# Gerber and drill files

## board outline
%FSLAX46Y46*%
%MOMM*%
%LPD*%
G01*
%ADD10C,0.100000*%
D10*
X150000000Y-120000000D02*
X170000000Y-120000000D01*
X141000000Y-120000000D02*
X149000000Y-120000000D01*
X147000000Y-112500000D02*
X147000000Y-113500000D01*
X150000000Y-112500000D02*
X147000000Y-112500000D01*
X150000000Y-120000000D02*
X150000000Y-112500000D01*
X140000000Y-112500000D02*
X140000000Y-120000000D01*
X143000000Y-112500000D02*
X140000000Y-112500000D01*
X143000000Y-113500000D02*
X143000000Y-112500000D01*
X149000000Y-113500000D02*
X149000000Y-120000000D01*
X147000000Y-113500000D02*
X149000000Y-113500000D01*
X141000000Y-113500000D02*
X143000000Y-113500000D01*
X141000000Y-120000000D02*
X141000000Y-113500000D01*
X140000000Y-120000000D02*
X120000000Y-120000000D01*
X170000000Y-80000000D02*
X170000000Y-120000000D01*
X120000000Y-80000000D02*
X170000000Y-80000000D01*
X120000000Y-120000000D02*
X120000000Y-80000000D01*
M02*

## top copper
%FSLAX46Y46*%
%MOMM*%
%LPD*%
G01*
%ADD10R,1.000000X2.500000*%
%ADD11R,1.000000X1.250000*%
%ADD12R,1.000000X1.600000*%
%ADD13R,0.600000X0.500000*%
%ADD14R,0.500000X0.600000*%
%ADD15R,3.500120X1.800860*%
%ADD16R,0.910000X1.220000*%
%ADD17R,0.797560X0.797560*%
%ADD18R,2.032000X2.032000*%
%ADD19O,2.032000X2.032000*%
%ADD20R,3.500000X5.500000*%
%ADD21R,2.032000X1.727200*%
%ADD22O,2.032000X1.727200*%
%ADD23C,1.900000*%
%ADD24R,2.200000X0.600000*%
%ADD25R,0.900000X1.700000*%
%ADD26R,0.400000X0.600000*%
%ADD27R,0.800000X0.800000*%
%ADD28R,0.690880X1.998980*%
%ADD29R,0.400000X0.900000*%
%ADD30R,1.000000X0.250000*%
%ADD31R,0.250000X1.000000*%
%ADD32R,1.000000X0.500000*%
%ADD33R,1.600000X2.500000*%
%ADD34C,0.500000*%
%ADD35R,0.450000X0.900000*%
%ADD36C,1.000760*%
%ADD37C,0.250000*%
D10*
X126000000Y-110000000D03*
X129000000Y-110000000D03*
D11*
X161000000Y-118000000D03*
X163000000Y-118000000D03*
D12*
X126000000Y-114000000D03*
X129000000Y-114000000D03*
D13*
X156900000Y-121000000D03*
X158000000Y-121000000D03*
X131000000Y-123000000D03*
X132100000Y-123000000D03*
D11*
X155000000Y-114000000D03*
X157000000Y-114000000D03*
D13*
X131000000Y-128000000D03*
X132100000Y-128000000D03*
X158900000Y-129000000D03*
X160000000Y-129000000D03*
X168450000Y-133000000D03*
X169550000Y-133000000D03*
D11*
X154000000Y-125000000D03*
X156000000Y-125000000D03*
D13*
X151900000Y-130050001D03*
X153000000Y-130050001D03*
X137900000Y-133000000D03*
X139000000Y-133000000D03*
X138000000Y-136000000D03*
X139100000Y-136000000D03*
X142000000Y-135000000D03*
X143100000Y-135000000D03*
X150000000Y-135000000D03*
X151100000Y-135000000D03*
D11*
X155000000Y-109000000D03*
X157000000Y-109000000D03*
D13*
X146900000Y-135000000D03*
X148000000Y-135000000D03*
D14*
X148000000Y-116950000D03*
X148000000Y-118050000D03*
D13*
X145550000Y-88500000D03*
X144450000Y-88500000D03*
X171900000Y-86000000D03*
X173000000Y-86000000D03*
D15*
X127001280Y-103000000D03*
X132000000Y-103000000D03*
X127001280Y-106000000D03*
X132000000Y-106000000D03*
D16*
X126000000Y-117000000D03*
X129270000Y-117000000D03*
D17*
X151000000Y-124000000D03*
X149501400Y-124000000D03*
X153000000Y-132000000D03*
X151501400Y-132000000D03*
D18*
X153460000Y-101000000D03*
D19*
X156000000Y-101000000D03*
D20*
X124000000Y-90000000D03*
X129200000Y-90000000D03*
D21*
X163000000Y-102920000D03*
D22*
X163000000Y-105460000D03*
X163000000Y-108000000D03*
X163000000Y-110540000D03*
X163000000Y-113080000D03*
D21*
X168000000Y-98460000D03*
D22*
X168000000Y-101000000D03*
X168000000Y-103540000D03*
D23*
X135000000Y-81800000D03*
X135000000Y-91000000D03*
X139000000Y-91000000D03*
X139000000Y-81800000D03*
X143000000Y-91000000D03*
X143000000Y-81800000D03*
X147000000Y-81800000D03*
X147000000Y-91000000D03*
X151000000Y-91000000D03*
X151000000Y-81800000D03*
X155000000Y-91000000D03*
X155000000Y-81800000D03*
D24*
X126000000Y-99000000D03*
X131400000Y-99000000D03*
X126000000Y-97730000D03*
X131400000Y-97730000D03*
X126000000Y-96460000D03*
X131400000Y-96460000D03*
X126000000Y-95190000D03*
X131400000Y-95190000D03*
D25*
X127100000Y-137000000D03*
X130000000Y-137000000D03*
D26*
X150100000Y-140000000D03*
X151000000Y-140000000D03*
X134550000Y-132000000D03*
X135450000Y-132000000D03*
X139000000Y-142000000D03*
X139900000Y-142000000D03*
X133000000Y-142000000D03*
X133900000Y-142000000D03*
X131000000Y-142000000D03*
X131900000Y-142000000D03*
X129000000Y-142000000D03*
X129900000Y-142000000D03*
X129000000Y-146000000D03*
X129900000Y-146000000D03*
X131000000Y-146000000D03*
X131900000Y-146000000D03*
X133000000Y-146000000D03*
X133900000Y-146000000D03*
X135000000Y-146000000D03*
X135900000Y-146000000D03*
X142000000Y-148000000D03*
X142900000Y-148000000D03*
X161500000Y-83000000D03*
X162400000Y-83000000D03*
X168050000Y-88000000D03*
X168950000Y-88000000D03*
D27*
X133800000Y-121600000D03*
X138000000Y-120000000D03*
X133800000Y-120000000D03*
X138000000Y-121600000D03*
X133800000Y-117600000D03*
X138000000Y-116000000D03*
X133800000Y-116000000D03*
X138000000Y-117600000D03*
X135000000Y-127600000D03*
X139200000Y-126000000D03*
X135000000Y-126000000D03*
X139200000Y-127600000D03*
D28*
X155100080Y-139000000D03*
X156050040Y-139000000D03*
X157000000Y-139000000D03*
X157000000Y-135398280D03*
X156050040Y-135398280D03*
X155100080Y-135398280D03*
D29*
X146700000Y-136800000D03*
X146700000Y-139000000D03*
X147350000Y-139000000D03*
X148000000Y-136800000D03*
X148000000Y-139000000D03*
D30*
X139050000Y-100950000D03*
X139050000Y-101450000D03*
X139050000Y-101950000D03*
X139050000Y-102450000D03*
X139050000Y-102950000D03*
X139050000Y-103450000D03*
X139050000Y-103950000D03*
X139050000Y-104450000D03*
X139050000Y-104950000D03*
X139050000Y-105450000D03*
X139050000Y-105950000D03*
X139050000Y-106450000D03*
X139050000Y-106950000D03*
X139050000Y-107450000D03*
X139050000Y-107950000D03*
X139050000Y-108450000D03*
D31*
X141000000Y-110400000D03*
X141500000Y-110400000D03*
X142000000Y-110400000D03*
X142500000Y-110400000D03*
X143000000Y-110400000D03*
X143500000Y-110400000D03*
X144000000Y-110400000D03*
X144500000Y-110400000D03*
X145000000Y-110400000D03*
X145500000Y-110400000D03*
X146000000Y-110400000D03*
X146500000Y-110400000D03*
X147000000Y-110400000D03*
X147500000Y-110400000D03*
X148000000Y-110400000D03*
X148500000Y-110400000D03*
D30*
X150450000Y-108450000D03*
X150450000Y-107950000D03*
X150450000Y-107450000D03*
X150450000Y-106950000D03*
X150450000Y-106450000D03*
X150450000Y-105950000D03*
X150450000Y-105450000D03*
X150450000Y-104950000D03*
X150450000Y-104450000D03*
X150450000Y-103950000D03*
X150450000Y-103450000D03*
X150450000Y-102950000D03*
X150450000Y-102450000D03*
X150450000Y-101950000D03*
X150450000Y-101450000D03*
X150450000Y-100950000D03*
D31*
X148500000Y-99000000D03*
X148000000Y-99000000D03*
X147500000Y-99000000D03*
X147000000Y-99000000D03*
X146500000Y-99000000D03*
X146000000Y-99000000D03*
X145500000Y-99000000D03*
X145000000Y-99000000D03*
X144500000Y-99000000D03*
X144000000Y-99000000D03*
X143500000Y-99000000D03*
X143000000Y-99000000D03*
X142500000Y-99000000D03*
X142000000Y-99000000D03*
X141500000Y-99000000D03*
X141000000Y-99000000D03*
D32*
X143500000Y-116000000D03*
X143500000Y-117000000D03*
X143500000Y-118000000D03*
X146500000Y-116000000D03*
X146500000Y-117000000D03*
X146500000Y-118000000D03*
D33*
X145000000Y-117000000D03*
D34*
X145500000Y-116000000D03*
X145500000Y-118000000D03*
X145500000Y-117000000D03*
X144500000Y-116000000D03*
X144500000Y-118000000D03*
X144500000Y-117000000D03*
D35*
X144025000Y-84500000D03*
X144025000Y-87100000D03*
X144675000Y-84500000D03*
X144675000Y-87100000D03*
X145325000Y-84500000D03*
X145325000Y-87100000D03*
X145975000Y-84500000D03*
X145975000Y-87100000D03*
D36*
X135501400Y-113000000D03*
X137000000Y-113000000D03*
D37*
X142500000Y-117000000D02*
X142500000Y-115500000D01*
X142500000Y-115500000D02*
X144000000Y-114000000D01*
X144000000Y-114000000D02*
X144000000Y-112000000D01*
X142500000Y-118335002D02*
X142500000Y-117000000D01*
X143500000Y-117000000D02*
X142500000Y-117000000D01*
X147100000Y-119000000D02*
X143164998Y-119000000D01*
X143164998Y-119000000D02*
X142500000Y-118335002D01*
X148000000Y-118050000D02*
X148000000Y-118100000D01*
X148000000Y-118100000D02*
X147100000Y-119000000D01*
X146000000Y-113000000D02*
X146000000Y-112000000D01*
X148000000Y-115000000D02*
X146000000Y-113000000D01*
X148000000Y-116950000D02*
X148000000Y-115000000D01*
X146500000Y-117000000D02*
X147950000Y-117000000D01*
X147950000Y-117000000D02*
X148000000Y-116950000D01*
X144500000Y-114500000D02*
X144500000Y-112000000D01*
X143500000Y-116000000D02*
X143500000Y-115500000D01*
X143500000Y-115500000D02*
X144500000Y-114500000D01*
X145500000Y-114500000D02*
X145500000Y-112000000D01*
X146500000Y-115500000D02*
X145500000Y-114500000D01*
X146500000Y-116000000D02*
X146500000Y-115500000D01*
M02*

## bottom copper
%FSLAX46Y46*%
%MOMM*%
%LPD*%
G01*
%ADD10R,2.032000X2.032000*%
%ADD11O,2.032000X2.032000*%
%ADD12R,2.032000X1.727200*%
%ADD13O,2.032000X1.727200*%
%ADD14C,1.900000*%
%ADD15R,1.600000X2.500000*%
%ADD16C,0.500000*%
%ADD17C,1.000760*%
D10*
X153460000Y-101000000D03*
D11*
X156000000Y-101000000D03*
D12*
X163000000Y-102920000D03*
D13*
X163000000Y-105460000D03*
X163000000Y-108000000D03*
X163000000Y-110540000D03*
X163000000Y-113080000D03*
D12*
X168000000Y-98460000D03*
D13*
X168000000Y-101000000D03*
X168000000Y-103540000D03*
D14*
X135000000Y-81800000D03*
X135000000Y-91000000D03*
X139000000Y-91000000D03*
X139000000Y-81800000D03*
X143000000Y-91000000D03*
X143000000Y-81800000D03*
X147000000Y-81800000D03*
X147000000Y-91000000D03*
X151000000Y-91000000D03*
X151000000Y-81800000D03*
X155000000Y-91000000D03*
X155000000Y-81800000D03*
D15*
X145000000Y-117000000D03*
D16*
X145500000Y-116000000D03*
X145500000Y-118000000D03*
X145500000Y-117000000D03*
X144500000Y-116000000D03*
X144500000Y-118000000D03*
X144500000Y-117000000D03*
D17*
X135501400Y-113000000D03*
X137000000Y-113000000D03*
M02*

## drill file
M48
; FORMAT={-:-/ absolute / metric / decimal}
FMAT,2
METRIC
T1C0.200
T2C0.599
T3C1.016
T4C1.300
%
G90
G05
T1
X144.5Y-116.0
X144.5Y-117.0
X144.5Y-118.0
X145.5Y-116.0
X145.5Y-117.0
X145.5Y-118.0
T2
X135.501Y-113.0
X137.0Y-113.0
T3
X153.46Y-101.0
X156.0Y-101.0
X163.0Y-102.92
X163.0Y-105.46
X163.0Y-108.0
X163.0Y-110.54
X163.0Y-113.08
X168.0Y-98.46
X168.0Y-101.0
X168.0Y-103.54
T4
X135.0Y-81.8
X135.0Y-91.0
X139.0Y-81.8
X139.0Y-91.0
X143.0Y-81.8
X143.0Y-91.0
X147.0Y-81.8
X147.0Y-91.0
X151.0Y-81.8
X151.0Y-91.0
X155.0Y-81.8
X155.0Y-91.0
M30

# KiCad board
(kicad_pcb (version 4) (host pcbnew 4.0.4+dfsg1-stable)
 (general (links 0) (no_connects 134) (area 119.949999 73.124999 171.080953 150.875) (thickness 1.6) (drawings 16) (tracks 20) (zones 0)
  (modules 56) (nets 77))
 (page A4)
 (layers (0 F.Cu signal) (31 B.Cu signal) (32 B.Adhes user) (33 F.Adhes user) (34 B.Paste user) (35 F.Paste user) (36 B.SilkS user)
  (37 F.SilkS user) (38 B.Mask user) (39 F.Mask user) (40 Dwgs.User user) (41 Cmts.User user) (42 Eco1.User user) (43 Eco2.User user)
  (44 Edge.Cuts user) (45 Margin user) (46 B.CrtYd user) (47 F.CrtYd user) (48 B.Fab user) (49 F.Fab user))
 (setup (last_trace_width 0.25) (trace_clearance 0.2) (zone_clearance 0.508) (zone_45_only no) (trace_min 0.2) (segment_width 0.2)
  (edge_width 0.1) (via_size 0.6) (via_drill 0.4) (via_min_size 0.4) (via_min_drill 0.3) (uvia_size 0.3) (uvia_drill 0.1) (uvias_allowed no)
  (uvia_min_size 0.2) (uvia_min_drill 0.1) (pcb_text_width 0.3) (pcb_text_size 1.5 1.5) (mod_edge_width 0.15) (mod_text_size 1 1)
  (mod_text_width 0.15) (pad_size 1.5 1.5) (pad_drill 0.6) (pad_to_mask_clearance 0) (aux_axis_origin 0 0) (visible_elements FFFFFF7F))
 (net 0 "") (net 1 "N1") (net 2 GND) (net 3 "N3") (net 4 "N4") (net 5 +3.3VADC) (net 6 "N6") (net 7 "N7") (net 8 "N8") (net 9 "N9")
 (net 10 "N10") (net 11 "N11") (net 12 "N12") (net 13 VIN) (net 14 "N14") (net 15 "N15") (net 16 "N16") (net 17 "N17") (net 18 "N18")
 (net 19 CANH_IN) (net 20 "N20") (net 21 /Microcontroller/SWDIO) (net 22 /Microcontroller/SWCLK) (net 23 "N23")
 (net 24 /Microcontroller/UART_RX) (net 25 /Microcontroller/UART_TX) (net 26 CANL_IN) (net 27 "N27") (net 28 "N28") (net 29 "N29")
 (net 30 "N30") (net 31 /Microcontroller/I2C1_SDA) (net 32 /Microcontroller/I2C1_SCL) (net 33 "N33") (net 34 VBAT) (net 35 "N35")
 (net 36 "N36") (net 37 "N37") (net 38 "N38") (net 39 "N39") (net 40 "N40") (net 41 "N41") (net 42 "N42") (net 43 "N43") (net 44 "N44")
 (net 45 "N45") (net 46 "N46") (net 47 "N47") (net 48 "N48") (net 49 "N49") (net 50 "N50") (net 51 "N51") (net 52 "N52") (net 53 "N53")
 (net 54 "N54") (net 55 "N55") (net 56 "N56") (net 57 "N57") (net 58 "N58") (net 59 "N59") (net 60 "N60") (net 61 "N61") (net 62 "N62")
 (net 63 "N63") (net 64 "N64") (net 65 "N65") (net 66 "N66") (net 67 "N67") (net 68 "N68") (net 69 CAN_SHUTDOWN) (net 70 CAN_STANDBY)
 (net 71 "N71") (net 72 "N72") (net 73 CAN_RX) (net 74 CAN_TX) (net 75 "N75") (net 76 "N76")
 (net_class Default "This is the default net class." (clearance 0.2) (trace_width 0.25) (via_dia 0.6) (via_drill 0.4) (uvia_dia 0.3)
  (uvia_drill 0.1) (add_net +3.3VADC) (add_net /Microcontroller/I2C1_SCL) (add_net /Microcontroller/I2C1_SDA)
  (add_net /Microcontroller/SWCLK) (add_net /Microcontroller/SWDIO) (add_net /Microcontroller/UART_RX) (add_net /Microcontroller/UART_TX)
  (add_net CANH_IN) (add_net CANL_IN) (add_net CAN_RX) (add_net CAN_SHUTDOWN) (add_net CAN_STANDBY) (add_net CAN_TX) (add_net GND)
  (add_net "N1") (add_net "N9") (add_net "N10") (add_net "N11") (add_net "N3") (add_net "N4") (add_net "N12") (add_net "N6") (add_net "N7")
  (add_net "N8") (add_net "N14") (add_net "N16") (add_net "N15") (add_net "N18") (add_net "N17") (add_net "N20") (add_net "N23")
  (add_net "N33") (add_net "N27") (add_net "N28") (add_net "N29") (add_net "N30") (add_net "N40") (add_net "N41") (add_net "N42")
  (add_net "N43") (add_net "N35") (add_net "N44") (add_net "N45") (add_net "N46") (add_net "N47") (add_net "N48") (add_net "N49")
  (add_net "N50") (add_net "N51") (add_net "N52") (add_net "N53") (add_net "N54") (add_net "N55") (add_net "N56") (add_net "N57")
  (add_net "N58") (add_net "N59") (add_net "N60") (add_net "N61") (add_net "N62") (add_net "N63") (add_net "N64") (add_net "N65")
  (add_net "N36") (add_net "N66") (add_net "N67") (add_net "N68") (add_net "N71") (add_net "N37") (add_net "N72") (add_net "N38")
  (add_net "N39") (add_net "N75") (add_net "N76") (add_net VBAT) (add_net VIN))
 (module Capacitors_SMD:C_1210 (layer F.Cu) (at 127.5 110)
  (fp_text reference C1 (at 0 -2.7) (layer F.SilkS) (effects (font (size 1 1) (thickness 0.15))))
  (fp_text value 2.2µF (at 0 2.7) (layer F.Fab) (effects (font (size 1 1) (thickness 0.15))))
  (pad 1 smd rect (at -1.5 0) (size 1 2.5) (layers F.Cu F.Paste F.Mask) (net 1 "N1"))
  (pad 2 smd rect (at 1.5 0) (size 1 2.5) (layers F.Cu F.Paste F.Mask) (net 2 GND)))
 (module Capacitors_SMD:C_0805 (layer F.Cu) (at 162 118)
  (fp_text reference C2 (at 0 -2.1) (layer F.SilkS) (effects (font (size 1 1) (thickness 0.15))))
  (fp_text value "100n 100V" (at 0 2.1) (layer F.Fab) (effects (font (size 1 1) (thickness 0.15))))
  (pad 1 smd rect (at -1 0) (size 1 1.25) (layers F.Cu F.Paste F.Mask) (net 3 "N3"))
  (pad 2 smd rect (at 1 0) (size 1 1.25) (layers F.Cu F.Paste F.Mask) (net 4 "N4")))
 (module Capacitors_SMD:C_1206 (layer F.Cu) (at 127.5 114)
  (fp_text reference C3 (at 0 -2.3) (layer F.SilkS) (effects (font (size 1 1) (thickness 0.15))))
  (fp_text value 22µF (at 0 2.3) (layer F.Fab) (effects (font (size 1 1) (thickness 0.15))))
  (pad 1 smd rect (at -1.5 0) (size 1 1.6) (layers F.Cu F.Paste F.Mask) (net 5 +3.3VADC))
  (pad 2 smd rect (at 1.5 0) (size 1 1.6) (layers F.Cu F.Paste F.Mask) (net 2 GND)))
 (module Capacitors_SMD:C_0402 (layer F.Cu) (at 157.45 121)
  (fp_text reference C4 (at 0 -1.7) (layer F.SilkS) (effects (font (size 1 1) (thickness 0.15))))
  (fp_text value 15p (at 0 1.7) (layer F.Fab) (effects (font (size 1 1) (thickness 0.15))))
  (pad 1 smd rect (at -0.55 0) (size 0.6 0.5) (layers F.Cu F.Paste F.Mask) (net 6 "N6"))
  (pad 2 smd rect (at 0.55 0) (size 0.6 0.5) (layers F.Cu F.Paste F.Mask) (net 2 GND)))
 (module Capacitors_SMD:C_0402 (layer F.Cu) (at 131.55 123)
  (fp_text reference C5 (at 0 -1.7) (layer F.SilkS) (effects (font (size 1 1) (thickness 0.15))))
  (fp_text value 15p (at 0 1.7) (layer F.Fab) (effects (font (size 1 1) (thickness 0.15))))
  (pad 1 smd rect (at -0.55 0) (size 0.6 0.5) (layers F.Cu F.Paste F.Mask) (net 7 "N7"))
  (pad 2 smd rect (at 0.55 0) (size 0.6 0.5) (layers F.Cu F.Paste F.Mask) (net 2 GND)))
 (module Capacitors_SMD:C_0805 (layer F.Cu) (at 156 114)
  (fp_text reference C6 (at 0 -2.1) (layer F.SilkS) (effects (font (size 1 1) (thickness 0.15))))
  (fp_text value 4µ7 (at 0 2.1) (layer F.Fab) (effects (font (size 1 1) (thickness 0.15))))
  (pad 1 smd rect (at -1 0) (size 1 1.25) (layers F.Cu F.Paste F.Mask) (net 5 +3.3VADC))
  (pad 2 smd rect (at 1 0) (size 1 1.25) (layers F.Cu F.Paste F.Mask) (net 2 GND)))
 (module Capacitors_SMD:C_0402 (layer F.Cu) (at 131.55 128)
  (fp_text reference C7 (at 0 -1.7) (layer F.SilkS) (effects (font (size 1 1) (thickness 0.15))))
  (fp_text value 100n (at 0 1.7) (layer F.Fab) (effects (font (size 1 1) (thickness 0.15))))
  (pad 1 smd rect (at -0.55 0) (size 0.6 0.5) (layers F.Cu F.Paste F.Mask) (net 5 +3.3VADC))
  (pad 2 smd rect (at 0.55 0) (size 0.6 0.5) (layers F.Cu F.Paste F.Mask) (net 2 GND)))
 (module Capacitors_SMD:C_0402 (layer F.Cu) (at 159.45 129)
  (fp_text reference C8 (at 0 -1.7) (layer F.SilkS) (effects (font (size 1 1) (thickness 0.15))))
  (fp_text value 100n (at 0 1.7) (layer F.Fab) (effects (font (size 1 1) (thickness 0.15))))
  (pad 1 smd rect (at -0.55 0) (size 0.6 0.5) (layers F.Cu F.Paste F.Mask) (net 5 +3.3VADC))
  (pad 2 smd rect (at 0.55 0) (size 0.6 0.5) (layers F.Cu F.Paste F.Mask) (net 2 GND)))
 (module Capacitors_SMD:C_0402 (layer F.Cu) (at 169 133)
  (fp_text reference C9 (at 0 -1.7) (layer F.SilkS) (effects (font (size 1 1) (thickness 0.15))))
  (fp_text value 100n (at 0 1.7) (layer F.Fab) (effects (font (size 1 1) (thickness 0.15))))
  (pad 1 smd rect (at -0.55 0) (size 0.6 0.5) (layers F.Cu F.Paste F.Mask) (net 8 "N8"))
  (pad 2 smd rect (at 0.55 0) (size 0.6 0.5) (layers F.Cu F.Paste F.Mask) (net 2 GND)))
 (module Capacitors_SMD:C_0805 (layer F.Cu) (at 155 125)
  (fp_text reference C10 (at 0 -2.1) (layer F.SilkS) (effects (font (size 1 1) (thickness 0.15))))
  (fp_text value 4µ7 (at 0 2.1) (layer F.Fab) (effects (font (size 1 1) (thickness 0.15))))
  (pad 1 smd rect (at -1 0) (size 1 1.25) (layers F.Cu F.Paste F.Mask) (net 5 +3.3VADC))
  (pad 2 smd rect (at 1 0) (size 1 1.25) (layers F.Cu F.Paste F.Mask) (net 2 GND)))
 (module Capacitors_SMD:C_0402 (layer F.Cu) (at 152.45 130.050001)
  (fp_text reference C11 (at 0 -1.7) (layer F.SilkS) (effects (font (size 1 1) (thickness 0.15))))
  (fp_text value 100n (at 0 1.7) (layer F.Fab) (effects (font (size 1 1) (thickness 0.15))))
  (pad 1 smd rect (at -0.55 0) (size 0.6 0.5) (layers F.Cu F.Paste F.Mask) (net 5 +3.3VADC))
  (pad 2 smd rect (at 0.55 0) (size 0.6 0.5) (layers F.Cu F.Paste F.Mask) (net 2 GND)))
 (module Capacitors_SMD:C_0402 (layer F.Cu) (at 138.45 133)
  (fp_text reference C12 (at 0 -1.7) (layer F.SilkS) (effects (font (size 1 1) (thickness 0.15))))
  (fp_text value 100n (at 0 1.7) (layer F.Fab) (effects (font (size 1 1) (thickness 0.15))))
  (pad 1 smd rect (at -0.55 0) (size 0.6 0.5) (layers F.Cu F.Paste F.Mask) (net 5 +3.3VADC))
  (pad 2 smd rect (at 0.55 0) (size 0.6 0.5) (layers F.Cu F.Paste F.Mask) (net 2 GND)))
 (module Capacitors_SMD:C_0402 (layer F.Cu) (at 138.55 136)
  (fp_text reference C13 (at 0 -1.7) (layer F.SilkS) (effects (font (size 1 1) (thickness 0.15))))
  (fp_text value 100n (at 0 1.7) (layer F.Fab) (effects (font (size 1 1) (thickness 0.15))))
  (pad 1 smd rect (at -0.55 0) (size 0.6 0.5) (layers F.Cu F.Paste F.Mask) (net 5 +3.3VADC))
  (pad 2 smd rect (at 0.55 0) (size 0.6 0.5) (layers F.Cu F.Paste F.Mask) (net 2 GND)))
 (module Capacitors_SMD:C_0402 (layer F.Cu) (at 142.55 135)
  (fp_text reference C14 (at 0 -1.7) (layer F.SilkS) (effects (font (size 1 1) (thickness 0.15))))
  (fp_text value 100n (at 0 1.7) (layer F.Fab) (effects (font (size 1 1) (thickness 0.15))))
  (pad 1 smd rect (at -0.55 0) (size 0.6 0.5) (layers F.Cu F.Paste F.Mask) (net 5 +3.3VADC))
  (pad 2 smd rect (at 0.55 0) (size 0.6 0.5) (layers F.Cu F.Paste F.Mask) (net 2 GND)))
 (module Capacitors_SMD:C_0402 (layer F.Cu) (at 150.55 135)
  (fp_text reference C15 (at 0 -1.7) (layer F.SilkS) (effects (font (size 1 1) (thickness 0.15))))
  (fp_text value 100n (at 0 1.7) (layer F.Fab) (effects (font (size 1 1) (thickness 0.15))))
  (pad 1 smd rect (at -0.55 0) (size 0.6 0.5) (layers F.Cu F.Paste F.Mask) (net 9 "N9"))
  (pad 2 smd rect (at 0.55 0) (size 0.6 0.5) (layers F.Cu F.Paste F.Mask) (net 2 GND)))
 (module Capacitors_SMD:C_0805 (layer F.Cu) (at 156 109)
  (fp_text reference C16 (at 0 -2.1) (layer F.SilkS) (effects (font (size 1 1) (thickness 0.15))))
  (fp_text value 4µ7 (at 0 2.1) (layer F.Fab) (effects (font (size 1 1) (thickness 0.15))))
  (pad 1 smd rect (at -1 0) (size 1 1.25) (layers F.Cu F.Paste F.Mask) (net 5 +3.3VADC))
  (pad 2 smd rect (at 1 0) (size 1 1.25) (layers F.Cu F.Paste F.Mask) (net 2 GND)))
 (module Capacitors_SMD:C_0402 (layer F.Cu) (at 147.45 135)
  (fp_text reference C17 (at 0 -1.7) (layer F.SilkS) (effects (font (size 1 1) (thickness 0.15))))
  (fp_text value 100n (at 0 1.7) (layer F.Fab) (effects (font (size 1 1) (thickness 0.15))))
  (pad 1 smd rect (at -0.55 0) (size 0.6 0.5) (layers F.Cu F.Paste F.Mask) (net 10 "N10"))
  (pad 2 smd rect (at 0.55 0) (size 0.6 0.5) (layers F.Cu F.Paste F.Mask) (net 2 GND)))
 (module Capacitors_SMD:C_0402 (layer F.Cu) (at 148 117.5 270)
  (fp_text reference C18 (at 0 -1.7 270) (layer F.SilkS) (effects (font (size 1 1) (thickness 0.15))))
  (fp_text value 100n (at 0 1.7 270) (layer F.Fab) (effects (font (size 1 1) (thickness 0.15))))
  (pad 1 smd rect (at -0.55 0 270) (size 0.6 0.5) (layers F.Cu F.Paste F.Mask) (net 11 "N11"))
  (pad 2 smd rect (at 0.55 0 270) (size 0.6 0.5) (layers F.Cu F.Paste F.Mask) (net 2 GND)))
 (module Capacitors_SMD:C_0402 (layer F.Cu) (at 145 88.5 180)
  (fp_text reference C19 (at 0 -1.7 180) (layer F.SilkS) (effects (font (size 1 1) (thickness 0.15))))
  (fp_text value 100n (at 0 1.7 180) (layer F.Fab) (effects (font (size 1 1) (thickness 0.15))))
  (pad 1 smd rect (at -0.55 0 180) (size 0.6 0.5) (layers F.Cu F.Paste F.Mask) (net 5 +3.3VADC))
  (pad 2 smd rect (at 0.55 0 180) (size 0.6 0.5) (layers F.Cu F.Paste F.Mask) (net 2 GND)))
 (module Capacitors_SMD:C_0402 (layer F.Cu) (at 172.45 86)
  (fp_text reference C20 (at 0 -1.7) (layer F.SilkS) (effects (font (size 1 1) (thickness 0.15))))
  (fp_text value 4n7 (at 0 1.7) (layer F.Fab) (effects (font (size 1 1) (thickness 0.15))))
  (pad 1 smd rect (at -0.55 0) (size 0.6 0.5) (layers F.Cu F.Paste F.Mask) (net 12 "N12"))
  (pad 2 smd rect (at 0.55 0) (size 0.6 0.5) (layers F.Cu F.Paste F.Mask) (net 2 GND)))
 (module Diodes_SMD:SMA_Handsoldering (layer F.Cu) (at 129.50064 103)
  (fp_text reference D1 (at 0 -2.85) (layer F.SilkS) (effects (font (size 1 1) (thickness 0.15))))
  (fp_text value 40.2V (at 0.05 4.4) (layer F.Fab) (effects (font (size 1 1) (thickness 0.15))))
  (pad 1 smd rect (at -2.49936 0) (size 3.50012 1.80086) (layers F.Cu F.Paste F.Mask) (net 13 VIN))
  (pad 2 smd rect (at 2.49936 0) (size 3.50012 1.80086) (layers F.Cu F.Paste F.Mask) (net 2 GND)))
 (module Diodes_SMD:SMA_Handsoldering (layer F.Cu) (at 129.50064 106)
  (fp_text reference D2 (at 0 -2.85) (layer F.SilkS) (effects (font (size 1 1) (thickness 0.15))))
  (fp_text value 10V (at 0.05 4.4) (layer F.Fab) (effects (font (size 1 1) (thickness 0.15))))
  (pad 1 smd rect (at -2.49936 0) (size 3.50012 1.80086) (layers F.Cu F.Paste F.Mask) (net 1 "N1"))
  (pad 2 smd rect (at 2.49936 0) (size 3.50012 1.80086) (layers F.Cu F.Paste F.Mask) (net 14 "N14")))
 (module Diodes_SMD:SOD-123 (layer F.Cu) (at 127.635 117)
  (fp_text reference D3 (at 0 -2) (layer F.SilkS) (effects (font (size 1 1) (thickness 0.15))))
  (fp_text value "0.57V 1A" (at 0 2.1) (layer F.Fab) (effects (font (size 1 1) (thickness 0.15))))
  (pad 1 smd rect (at -1.635 0) (size 0.91 1.22) (layers F.Cu F.Paste F.Mask) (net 3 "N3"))
  (pad 2 smd rect (at 1.635 0) (size 0.91 1.22) (layers F.Cu F.Paste F.Mask) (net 2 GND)))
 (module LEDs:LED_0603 (layer F.Cu) (at 150.2507 124)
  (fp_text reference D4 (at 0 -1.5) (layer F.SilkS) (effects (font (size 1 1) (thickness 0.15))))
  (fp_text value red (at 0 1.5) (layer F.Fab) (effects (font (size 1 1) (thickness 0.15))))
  (pad 2 smd rect (at 0.7493 0 180) (size 0.79756 0.79756) (layers F.Cu F.Paste F.Mask) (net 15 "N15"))
  (pad 1 smd rect (at -0.7493 0 180) (size 0.79756 0.79756) (layers F.Cu F.Paste F.Mask) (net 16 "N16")))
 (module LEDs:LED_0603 (layer F.Cu) (at 152.2507 132)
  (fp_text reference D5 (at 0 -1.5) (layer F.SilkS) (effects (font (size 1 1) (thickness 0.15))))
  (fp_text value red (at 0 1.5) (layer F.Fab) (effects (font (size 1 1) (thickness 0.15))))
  (pad 2 smd rect (at 0.7493 0 180) (size 0.79756 0.79756) (layers F.Cu F.Paste F.Mask) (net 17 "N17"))
  (pad 1 smd rect (at -0.7493 0 180) (size 0.79756 0.79756) (layers F.Cu F.Paste F.Mask) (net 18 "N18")))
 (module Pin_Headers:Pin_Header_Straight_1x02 (layer F.Cu) (at 153.46 101 90)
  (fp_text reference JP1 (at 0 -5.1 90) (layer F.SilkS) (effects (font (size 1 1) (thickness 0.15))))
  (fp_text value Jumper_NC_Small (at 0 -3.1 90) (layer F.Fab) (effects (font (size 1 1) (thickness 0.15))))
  (pad 1 thru_hole rect (at 0 0 90) (size 2.032 2.032) (drill 1.016) (layers *.Cu *.Mask F.SilkS) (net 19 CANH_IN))
  (pad 2 thru_hole oval (at 0 2.54 90) (size 2.032 2.032) (drill 1.016) (layers *.Cu *.Mask F.SilkS) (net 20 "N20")))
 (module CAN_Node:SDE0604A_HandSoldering (layer F.Cu) (at 126.6 90)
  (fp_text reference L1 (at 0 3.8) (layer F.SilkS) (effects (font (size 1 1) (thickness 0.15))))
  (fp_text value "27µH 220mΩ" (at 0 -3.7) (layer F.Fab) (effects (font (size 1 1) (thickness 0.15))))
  (pad 1 smd rect (at -2.6 0) (size 3.5 5.5) (layers F.Cu F.Paste F.Mask) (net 3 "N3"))
  (pad 2 smd rect (at 2.6 0) (size 3.5 5.5) (layers F.Cu F.Paste F.Mask) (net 5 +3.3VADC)))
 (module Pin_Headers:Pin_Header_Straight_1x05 (layer F.Cu) (at 163 102.92)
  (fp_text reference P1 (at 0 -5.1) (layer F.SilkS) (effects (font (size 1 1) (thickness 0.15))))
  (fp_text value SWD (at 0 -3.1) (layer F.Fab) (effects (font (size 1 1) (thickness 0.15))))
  (pad 1 thru_hole rect (at 0 0) (size 2.032 1.7272) (drill 1.016) (layers *.Cu *.Mask F.SilkS) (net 5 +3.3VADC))
  (pad 2 thru_hole oval (at 0 2.54) (size 2.032 1.7272) (drill 1.016) (layers *.Cu *.Mask F.SilkS) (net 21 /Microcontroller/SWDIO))
  (pad 3 thru_hole oval (at 0 5.08) (size 2.032 1.7272) (drill 1.016) (layers *.Cu *.Mask F.SilkS) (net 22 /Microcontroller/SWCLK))
  (pad 4 thru_hole oval (at 0 7.62) (size 2.032 1.7272) (drill 1.016) (layers *.Cu *.Mask F.SilkS) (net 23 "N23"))
  (pad 5 thru_hole oval (at 0 10.16) (size 2.032 1.7272) (drill 1.016) (layers *.Cu *.Mask F.SilkS) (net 2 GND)))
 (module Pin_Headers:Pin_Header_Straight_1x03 (layer F.Cu) (at 168 98.46)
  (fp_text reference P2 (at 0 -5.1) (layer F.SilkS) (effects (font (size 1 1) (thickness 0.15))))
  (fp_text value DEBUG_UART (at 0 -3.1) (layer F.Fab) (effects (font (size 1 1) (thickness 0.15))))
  (pad 1 thru_hole rect (at 0 0) (size 2.032 1.7272) (drill 1.016) (layers *.Cu *.Mask F.SilkS) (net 2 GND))
  (pad 2 thru_hole oval (at 0 2.54) (size 2.032 1.7272) (drill 1.016) (layers *.Cu *.Mask F.SilkS) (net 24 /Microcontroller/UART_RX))
  (pad 3 thru_hole oval (at 0 5.08) (size 2.032 1.7272) (drill 1.016) (layers *.Cu *.Mask F.SilkS) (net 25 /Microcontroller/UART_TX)))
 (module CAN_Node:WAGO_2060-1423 (layer B.Cu) (at 139 86.4)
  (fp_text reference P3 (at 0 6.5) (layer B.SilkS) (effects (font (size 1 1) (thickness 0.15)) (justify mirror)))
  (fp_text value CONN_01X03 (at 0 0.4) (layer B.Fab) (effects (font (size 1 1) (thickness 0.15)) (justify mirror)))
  (pad 1 thru_hole circle (at -4 -4.6) (size 1.9 1.9) (drill 1.3) (layers *.Cu *.Mask) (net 13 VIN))
  (pad 1 thru_hole circle (at -4 4.6) (size 1.9 1.9) (drill 1.3) (layers *.Cu *.Mask) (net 13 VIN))
  (pad 2 thru_hole circle (at 0 4.6) (size 1.9 1.9) (drill 1.3) (layers *.Cu *.Mask) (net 2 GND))
  (pad 2 thru_hole circle (at 0 -4.6) (size 1.9 1.9) (drill 1.3) (layers *.Cu *.Mask) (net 2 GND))
  (pad 3 thru_hole circle (at 4 4.6) (size 1.9 1.9) (drill 1.3) (layers *.Cu *.Mask) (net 19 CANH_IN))
  (pad 3 thru_hole circle (at 4 -4.6) (size 1.9 1.9) (drill 1.3) (layers *.Cu *.Mask) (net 19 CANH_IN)))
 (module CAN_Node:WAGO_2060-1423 (layer B.Cu) (at 151 86.4)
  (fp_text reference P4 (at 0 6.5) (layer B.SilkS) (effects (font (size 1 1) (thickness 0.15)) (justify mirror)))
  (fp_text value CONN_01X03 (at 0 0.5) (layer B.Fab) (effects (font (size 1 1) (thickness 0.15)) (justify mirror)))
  (pad 1 thru_hole circle (at -4 -4.6) (size 1.9 1.9) (drill 1.3) (layers *.Cu *.Mask) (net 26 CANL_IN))
  (pad 1 thru_hole circle (at -4 4.6) (size 1.9 1.9) (drill 1.3) (layers *.Cu *.Mask) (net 26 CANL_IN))
  (pad 2 thru_hole circle (at 0 4.6) (size 1.9 1.9) (drill 1.3) (layers *.Cu *.Mask) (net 19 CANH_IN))
  (pad 2 thru_hole circle (at 0 -4.6) (size 1.9 1.9) (drill 1.3) (layers *.Cu *.Mask) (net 19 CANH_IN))
  (pad 3 thru_hole circle (at 4 4.6) (size 1.9 1.9) (drill 1.3) (layers *.Cu *.Mask) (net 26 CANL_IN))
  (pad 3 thru_hole circle (at 4 -4.6) (size 1.9 1.9) (drill 1.3) (layers *.Cu *.Mask) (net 26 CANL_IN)))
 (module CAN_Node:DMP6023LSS (layer F.Cu) (at 128.7 97.095 90)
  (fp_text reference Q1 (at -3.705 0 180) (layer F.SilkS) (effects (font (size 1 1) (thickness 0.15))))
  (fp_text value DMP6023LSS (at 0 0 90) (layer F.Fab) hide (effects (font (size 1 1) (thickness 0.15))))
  (pad 5 smd rect (at -1.905 -2.7 90) (size 0.6 2.2) (layers F.Cu F.Paste F.Mask) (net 13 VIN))
  (pad 1 smd rect (at -1.905 2.7 90) (size 0.6 2.2) (layers F.Cu F.Paste F.Mask) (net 1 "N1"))
  (pad 5 smd rect (at -0.635 -2.7 90) (size 0.6 2.2) (layers F.Cu F.Paste F.Mask) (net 13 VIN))
  (pad 1 smd rect (at -0.635 2.7 90) (size 0.6 2.2) (layers F.Cu F.Paste F.Mask) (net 1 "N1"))
  (pad 5 smd rect (at 0.635 -2.7 90) (size 0.6 2.2) (layers F.Cu F.Paste F.Mask) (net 13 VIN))
  (pad 1 smd rect (at 0.635 2.7 90) (size 0.6 2.2) (layers F.Cu F.Paste F.Mask) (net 1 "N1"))
  (pad 5 smd rect (at 1.905 -2.7 90) (size 0.6 2.2) (layers F.Cu F.Paste F.Mask) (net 13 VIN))
  (pad 4 smd rect (at 1.905 2.7 90) (size 0.6 2.2) (layers F.Cu F.Paste F.Mask) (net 14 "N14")))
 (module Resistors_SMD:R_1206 (layer F.Cu) (at 128.55 137)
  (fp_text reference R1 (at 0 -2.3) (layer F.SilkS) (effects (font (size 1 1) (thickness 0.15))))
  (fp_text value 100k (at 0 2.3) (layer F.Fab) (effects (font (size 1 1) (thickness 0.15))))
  (pad 1 smd rect (at -1.45 0) (size 0.9 1.7) (layers F.Cu F.Paste F.Mask) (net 14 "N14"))
  (pad 2 smd rect (at 1.45 0) (size 0.9 1.7) (layers F.Cu F.Paste F.Mask) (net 2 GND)))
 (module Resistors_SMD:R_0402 (layer F.Cu) (at 150.55 140)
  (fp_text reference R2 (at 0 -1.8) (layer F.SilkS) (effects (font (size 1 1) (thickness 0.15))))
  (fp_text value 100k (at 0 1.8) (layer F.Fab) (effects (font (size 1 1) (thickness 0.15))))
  (pad 1 smd rect (at -0.45 0) (size 0.4 0.6) (layers F.Cu F.Paste F.Mask) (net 1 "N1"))
  (pad 2 smd rect (at 0.45 0) (size 0.4 0.6) (layers F.Cu F.Paste F.Mask) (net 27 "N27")))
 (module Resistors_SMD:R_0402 (layer F.Cu) (at 135 132)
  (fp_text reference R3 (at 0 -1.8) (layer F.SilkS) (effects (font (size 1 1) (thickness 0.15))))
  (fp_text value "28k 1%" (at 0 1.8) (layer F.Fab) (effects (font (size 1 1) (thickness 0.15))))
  (pad 1 smd rect (at -0.45 0) (size 0.4 0.6) (layers F.Cu F.Paste F.Mask) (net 5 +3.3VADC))
  (pad 2 smd rect (at 0.45 0) (size 0.4 0.6) (layers F.Cu F.Paste F.Mask) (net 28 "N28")))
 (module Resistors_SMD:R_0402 (layer F.Cu) (at 139.45 142)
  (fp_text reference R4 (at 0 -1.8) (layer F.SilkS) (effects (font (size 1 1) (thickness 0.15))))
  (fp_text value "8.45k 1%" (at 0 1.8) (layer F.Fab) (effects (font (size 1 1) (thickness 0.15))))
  (pad 1 smd rect (at -0.45 0) (size 0.4 0.6) (layers F.Cu F.Paste F.Mask) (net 28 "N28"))
  (pad 2 smd rect (at 0.45 0) (size 0.4 0.6) (layers F.Cu F.Paste F.Mask) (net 2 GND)))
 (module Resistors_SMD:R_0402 (layer F.Cu) (at 133.45 142)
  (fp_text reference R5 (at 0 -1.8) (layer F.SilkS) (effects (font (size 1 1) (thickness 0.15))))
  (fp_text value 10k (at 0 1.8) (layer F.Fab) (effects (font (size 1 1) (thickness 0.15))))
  (pad 1 smd rect (at -0.45 0) (size 0.4 0.6) (layers F.Cu F.Paste F.Mask) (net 5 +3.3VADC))
  (pad 2 smd rect (at 0.45 0) (size 0.4 0.6) (layers F.Cu F.Paste F.Mask) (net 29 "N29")))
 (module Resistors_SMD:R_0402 (layer F.Cu) (at 131.45 142)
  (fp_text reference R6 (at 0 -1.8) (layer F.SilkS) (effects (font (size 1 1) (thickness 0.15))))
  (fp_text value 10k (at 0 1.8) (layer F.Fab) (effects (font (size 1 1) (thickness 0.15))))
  (pad 1 smd rect (at -0.45 0) (size 0.4 0.6) (layers F.Cu F.Paste F.Mask) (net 5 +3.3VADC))
  (pad 2 smd rect (at 0.45 0) (size 0.4 0.6) (layers F.Cu F.Paste F.Mask) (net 23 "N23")))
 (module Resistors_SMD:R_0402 (layer F.Cu) (at 129.45 142)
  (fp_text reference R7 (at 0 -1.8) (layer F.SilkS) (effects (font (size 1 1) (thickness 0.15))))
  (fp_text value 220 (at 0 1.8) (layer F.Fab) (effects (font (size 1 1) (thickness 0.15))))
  (pad 1 smd rect (at -0.45 0) (size 0.4 0.6) (layers F.Cu F.Paste F.Mask) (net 2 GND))
  (pad 2 smd rect (at 0.45 0) (size 0.4 0.6) (layers F.Cu F.Paste F.Mask) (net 16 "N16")))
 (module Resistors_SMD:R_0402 (layer F.Cu) (at 129.45 146)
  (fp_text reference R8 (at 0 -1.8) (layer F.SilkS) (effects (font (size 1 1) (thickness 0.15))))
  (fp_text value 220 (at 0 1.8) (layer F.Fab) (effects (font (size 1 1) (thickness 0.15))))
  (pad 1 smd rect (at -0.45 0) (size 0.4 0.6) (layers F.Cu F.Paste F.Mask) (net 2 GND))
  (pad 2 smd rect (at 0.45 0) (size 0.4 0.6) (layers F.Cu F.Paste F.Mask) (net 18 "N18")))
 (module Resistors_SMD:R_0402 (layer F.Cu) (at 131.45 146)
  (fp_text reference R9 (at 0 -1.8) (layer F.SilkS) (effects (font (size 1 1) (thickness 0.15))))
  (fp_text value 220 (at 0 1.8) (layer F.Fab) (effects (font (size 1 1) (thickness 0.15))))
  (pad 1 smd rect (at -0.45 0) (size 0.4 0.6) (layers F.Cu F.Paste F.Mask) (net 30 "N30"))
  (pad 2 smd rect (at 0.45 0) (size 0.4 0.6) (layers F.Cu F.Paste F.Mask) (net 9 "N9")))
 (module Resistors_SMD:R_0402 (layer F.Cu) (at 133.45 146)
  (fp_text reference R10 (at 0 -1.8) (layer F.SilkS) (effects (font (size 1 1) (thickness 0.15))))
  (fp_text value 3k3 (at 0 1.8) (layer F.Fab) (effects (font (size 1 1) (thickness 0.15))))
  (pad 1 smd rect (at -0.45 0) (size 0.4 0.6) (layers F.Cu F.Paste F.Mask) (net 5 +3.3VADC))
  (pad 2 smd rect (at 0.45 0) (size 0.4 0.6) (layers F.Cu F.Paste F.Mask) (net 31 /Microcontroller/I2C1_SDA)))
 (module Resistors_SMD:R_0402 (layer F.Cu) (at 135.45 146)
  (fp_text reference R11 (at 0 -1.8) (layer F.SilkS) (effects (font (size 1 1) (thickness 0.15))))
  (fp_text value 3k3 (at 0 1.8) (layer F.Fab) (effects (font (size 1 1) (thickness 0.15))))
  (pad 1 smd rect (at -0.45 0) (size 0.4 0.6) (layers F.Cu F.Paste F.Mask) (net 5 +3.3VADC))
  (pad 2 smd rect (at 0.45 0) (size 0.4 0.6) (layers F.Cu F.Paste F.Mask) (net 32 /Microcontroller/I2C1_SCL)))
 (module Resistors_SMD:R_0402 (layer F.Cu) (at 142.45 148)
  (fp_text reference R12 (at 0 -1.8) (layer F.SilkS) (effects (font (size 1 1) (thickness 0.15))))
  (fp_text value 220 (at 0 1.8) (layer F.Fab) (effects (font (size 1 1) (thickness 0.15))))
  (pad 1 smd rect (at -0.45 0) (size 0.4 0.6) (layers F.Cu F.Paste F.Mask) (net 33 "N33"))
  (pad 2 smd rect (at 0.45 0) (size 0.4 0.6) (layers F.Cu F.Paste F.Mask) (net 10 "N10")))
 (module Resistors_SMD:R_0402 (layer F.Cu) (at 161.95 83)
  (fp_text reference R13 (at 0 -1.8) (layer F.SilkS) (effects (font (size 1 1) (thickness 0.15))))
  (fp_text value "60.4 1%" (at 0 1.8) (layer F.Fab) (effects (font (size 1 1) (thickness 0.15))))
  (pad 1 smd rect (at -0.45 0) (size 0.4 0.6) (layers F.Cu F.Paste F.Mask) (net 20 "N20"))
  (pad 2 smd rect (at 0.45 0) (size 0.4 0.6) (layers F.Cu F.Paste F.Mask) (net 12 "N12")))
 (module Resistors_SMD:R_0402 (layer F.Cu) (at 168.5 88)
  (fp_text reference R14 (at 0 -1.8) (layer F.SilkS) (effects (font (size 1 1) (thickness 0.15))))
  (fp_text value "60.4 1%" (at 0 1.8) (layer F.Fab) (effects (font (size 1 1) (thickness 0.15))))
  (pad 1 smd rect (at -0.45 0) (size 0.4 0.6) (layers F.Cu F.Paste F.Mask) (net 12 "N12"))
  (pad 2 smd rect (at 0.45 0) (size 0.4 0.6) (layers F.Cu F.Paste F.Mask) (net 26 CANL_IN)))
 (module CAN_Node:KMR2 (layer F.Cu) (at 135.9 120.8)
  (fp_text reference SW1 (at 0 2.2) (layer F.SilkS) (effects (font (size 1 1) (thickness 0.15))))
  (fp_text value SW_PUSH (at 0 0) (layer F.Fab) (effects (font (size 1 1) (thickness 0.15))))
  (pad 1 smd rect (at -2.1 0.8) (size 0.8 0.8) (layers F.Cu F.Paste F.Mask) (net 29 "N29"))
  (pad 2 smd rect (at 2.1 -0.8) (size 0.8 0.8) (layers F.Cu F.Paste F.Mask) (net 2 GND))
  (pad 2 smd rect (at -2.1 -0.8) (size 0.8 0.8) (layers F.Cu F.Paste F.Mask) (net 2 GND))
  (pad 1 smd rect (at 2.1 0.8) (size 0.8 0.8) (layers F.Cu F.Paste F.Mask) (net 29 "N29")))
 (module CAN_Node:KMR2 (layer F.Cu) (at 135.9 116.8)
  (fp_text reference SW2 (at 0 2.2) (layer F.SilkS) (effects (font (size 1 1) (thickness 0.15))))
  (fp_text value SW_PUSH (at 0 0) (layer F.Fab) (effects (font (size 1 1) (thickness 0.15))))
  (pad 1 smd rect (at -2.1 0.8) (size 0.8 0.8) (layers F.Cu F.Paste F.Mask) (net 2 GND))
  (pad 2 smd rect (at 2.1 -0.8) (size 0.8 0.8) (layers F.Cu F.Paste F.Mask) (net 30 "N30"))
  (pad 2 smd rect (at -2.1 -0.8) (size 0.8 0.8) (layers F.Cu F.Paste F.Mask) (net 30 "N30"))
  (pad 1 smd rect (at 2.1 0.8) (size 0.8 0.8) (layers F.Cu F.Paste F.Mask) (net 2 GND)))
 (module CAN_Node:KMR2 (layer F.Cu) (at 137.1 126.8)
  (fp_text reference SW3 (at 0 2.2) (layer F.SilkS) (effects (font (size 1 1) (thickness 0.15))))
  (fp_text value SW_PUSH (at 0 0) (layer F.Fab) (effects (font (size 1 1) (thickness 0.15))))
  (pad 1 smd rect (at -2.1 0.8) (size 0.8 0.8) (layers F.Cu F.Paste F.Mask) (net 2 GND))
  (pad 2 smd rect (at 2.1 -0.8) (size 0.8 0.8) (layers F.Cu F.Paste F.Mask) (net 33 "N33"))
  (pad 2 smd rect (at -2.1 -0.8) (size 0.8 0.8) (layers F.Cu F.Paste F.Mask) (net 33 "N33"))
  (pad 1 smd rect (at 2.1 0.8) (size 0.8 0.8) (layers F.Cu F.Paste F.Mask) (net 2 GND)))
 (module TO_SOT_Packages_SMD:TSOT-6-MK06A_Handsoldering (layer F.Cu) (at 156.05004 137.19914)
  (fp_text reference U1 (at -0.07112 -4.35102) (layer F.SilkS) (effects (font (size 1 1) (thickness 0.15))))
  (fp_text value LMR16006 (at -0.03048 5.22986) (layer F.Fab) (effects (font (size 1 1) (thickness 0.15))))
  (pad 1 smd rect (at -0.94996 1.80086) (size 0.69088 1.99898) (layers F.Cu F.Paste F.Mask) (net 4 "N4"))
  (pad 2 smd rect (at 0 1.80086) (size 0.69088 1.99898) (layers F.Cu F.Paste F.Mask) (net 2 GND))
  (pad 3 smd rect (at 0.94996 1.80086) (size 0.69088 1.99898) (layers F.Cu F.Paste F.Mask) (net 28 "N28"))
  (pad 4 smd rect (at 0.94996 -1.80086) (size 0.69088 1.99898) (layers F.Cu F.Paste F.Mask) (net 27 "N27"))
  (pad 5 smd rect (at 0 -1.80086) (size 0.69088 1.99898) (layers F.Cu F.Paste F.Mask) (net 1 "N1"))
  (pad 6 smd rect (at -0.94996 -1.80086) (size 0.69088 1.99898) (layers F.Cu F.Paste F.Mask) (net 3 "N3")))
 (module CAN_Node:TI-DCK (layer F.Cu) (at 147.35 137.9)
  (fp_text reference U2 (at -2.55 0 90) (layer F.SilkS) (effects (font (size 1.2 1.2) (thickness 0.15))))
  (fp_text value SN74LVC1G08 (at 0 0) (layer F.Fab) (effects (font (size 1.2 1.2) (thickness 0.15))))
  (pad 5 smd rect (at -0.65 -1.1) (size 0.4 0.9) (layers F.Cu F.Paste F.Mask) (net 5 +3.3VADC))
  (pad 1 smd rect (at -0.65 1.1) (size 0.4 0.9) (layers F.Cu F.Paste F.Mask) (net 29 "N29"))
  (pad 2 smd rect (at 0 1.1) (size 0.4 0.9) (layers F.Cu F.Paste F.Mask) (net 23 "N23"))
  (pad 4 smd rect (at 0.65 -1.1) (size 0.4 0.9) (layers F.Cu F.Paste F.Mask) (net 8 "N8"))
  (pad 3 smd rect (at 0.65 1.1) (size 0.4 0.9) (layers F.Cu F.Paste F.Mask) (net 2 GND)))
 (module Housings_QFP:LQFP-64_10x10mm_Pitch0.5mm (layer F.Cu) (at 144.75 104.7)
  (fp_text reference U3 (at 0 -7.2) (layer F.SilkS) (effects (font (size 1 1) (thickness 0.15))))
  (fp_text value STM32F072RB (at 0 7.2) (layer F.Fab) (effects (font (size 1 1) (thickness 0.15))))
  (pad 1 smd rect (at -5.7 -3.75) (size 1 0.25) (layers F.Cu F.Paste F.Mask) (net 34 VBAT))
  (pad 2 smd rect (at -5.7 -3.25) (size 1 0.25) (layers F.Cu F.Paste F.Mask) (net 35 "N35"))
  (pad 3 smd rect (at -5.7 -2.75) (size 1 0.25) (layers F.Cu F.Paste F.Mask) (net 6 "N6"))
  (pad 4 smd rect (at -5.7 -2.25) (size 1 0.25) (layers F.Cu F.Paste F.Mask) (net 7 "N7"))
  (pad 5 smd rect (at -5.7 -1.75) (size 1 0.25) (layers F.Cu F.Paste F.Mask) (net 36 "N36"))
  (pad 6 smd rect (at -5.7 -1.25) (size 1 0.25) (layers F.Cu F.Paste F.Mask) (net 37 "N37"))
  (pad 7 smd rect (at -5.7 -0.75) (size 1 0.25) (layers F.Cu F.Paste F.Mask) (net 8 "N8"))
  (pad 8 smd rect (at -5.7 -0.25) (size 1 0.25) (layers F.Cu F.Paste F.Mask) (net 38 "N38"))
  (pad 9 smd rect (at -5.7 0.25) (size 1 0.25) (layers F.Cu F.Paste F.Mask) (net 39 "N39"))
  (pad 10 smd rect (at -5.7 0.75) (size 1 0.25) (layers F.Cu F.Paste F.Mask) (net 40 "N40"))
  (pad 11 smd rect (at -5.7 1.25) (size 1 0.25) (layers F.Cu F.Paste F.Mask) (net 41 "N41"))
  (pad 12 smd rect (at -5.7 1.75) (size 1 0.25) (layers F.Cu F.Paste F.Mask) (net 2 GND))
  (pad 13 smd rect (at -5.7 2.25) (size 1 0.25) (layers F.Cu F.Paste F.Mask) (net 5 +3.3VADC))
  (pad 14 smd rect (at -5.7 2.75) (size 1 0.25) (layers F.Cu F.Paste F.Mask) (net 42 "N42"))
  (pad 15 smd rect (at -5.7 3.25) (size 1 0.25) (layers F.Cu F.Paste F.Mask) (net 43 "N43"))
  (pad 16 smd rect (at -5.7 3.75) (size 1 0.25) (layers F.Cu F.Paste F.Mask) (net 25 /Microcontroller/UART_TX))
  (pad 17 smd rect (at -3.75 5.7 90) (size 1 0.25) (layers F.Cu F.Paste F.Mask) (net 24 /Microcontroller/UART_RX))
  (pad 18 smd rect (at -3.25 5.7 90) (size 1 0.25) (layers F.Cu F.Paste F.Mask) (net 2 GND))
  (pad 19 smd rect (at -2.75 5.7 90) (size 1 0.25) (layers F.Cu F.Paste F.Mask) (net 5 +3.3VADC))
  (pad 20 smd rect (at -2.25 5.7 90) (size 1 0.25) (layers F.Cu F.Paste F.Mask) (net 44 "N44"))
  (pad 21 smd rect (at -1.75 5.7 90) (size 1 0.25) (layers F.Cu F.Paste F.Mask) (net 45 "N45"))
  (pad 22 smd rect (at -1.25 5.7 90) (size 1 0.25) (layers F.Cu F.Paste F.Mask) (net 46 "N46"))
  (pad 23 smd rect (at -0.75 5.7 90) (size 1 0.25) (layers F.Cu F.Paste F.Mask) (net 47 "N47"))
  (pad 24 smd rect (at -0.25 5.7 90) (size 1 0.25) (layers F.Cu F.Paste F.Mask) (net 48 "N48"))
  (pad 25 smd rect (at 0.25 5.7 90) (size 1 0.25) (layers F.Cu F.Paste F.Mask) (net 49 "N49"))
  (pad 26 smd rect (at 0.75 5.7 90) (size 1 0.25) (layers F.Cu F.Paste F.Mask) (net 15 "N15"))
  (pad 27 smd rect (at 1.25 5.7 90) (size 1 0.25) (layers F.Cu F.Paste F.Mask) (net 17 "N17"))
  (pad 28 smd rect (at 1.75 5.7 90) (size 1 0.25) (layers F.Cu F.Paste F.Mask) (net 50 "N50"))
  (pad 29 smd rect (at 2.25 5.7 90) (size 1 0.25) (layers F.Cu F.Paste F.Mask) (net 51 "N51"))
  (pad 30 smd rect (at 2.75 5.7 90) (size 1 0.25) (layers F.Cu F.Paste F.Mask) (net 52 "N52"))
  (pad 31 smd rect (at 3.25 5.7 90) (size 1 0.25) (layers F.Cu F.Paste F.Mask) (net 2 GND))
  (pad 32 smd rect (at 3.75 5.7 90) (size 1 0.25) (layers F.Cu F.Paste F.Mask) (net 5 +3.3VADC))
  (pad 33 smd rect (at 5.7 3.75) (size 1 0.25) (layers F.Cu F.Paste F.Mask) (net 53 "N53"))
  (pad 34 smd rect (at 5.7 3.25) (size 1 0.25) (layers F.Cu F.Paste F.Mask) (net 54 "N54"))
  (pad 35 smd rect (at 5.7 2.75) (size 1 0.25) (layers F.Cu F.Paste F.Mask) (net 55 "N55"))
  (pad 36 smd rect (at 5.7 2.25) (size 1 0.25) (layers F.Cu F.Paste F.Mask) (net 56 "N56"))
  (pad 37 smd rect (at 5.7 1.75) (size 1 0.25) (layers F.Cu F.Paste F.Mask) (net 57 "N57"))
  (pad 38 smd rect (at 5.7 1.25) (size 1 0.25) (layers F.Cu F.Paste F.Mask) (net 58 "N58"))
  (pad 39 smd rect (at 5.7 0.75) (size 1 0.25) (layers F.Cu F.Paste F.Mask) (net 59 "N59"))
  (pad 40 smd rect (at 5.7 0.25) (size 1 0.25) (layers F.Cu F.Paste F.Mask) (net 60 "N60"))
  (pad 41 smd rect (at 5.7 -0.25) (size 1 0.25) (layers F.Cu F.Paste F.Mask) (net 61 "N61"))
  (pad 42 smd rect (at 5.7 -0.75) (size 1 0.25) (layers F.Cu F.Paste F.Mask) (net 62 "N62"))
  (pad 43 smd rect (at 5.7 -1.25) (size 1 0.25) (layers F.Cu F.Paste F.Mask) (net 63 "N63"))
  (pad 44 smd rect (at 5.7 -1.75) (size 1 0.25) (layers F.Cu F.Paste F.Mask) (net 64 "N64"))
  (pad 45 smd rect (at 5.7 -2.25) (size 1 0.25) (layers F.Cu F.Paste F.Mask) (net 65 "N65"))
  (pad 46 smd rect (at 5.7 -2.75) (size 1 0.25) (layers F.Cu F.Paste F.Mask) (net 21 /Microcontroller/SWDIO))
  (pad 47 smd rect (at 5.7 -3.25) (size 1 0.25) (layers F.Cu F.Paste F.Mask) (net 2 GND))
  (pad 48 smd rect (at 5.7 -3.75) (size 1 0.25) (layers F.Cu F.Paste F.Mask) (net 5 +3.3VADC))
  (pad 49 smd rect (at 3.75 -5.7 90) (size 1 0.25) (layers F.Cu F.Paste F.Mask) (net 22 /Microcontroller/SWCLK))
  (pad 50 smd rect (at 3.25 -5.7 90) (size 1 0.25) (layers F.Cu F.Paste F.Mask) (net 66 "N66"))
  (pad 51 smd rect (at 2.75 -5.7 90) (size 1 0.25) (layers F.Cu F.Paste F.Mask) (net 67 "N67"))
  (pad 52 smd rect (at 2.25 -5.7 90) (size 1 0.25) (layers F.Cu F.Paste F.Mask) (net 9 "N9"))
  (pad 53 smd rect (at 1.75 -5.7 90) (size 1 0.25) (layers F.Cu F.Paste F.Mask) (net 10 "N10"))
  (pad 54 smd rect (at 1.25 -5.7 90) (size 1 0.25) (layers F.Cu F.Paste F.Mask) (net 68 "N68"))
  (pad 55 smd rect (at 0.75 -5.7 90) (size 1 0.25) (layers F.Cu F.Paste F.Mask) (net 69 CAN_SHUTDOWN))
  (pad 56 smd rect (at 0.25 -5.7 90) (size 1 0.25) (layers F.Cu F.Paste F.Mask) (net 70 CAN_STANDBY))
  (pad 57 smd rect (at -0.25 -5.7 90) (size 1 0.25) (layers F.Cu F.Paste F.Mask) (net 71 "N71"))
  (pad 58 smd rect (at -0.75 -5.7 90) (size 1 0.25) (layers F.Cu F.Paste F.Mask) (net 32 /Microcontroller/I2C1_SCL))
  (pad 59 smd rect (at -1.25 -5.7 90) (size 1 0.25) (layers F.Cu F.Paste F.Mask) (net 31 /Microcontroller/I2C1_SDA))
  (pad 60 smd rect (at -1.75 -5.7 90) (size 1 0.25) (layers F.Cu F.Paste F.Mask) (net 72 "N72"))
  (pad 61 smd rect (at -2.25 -5.7 90) (size 1 0.25) (layers F.Cu F.Paste F.Mask) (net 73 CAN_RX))
  (pad 62 smd rect (at -2.75 -5.7 90) (size 1 0.25) (layers F.Cu F.Paste F.Mask) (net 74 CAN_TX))
  (pad 63 smd rect (at -3.25 -5.7 90) (size 1 0.25) (layers F.Cu F.Paste F.Mask) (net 2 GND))
  (pad 64 smd rect (at -3.75 -5.7 90) (size 1 0.25) (layers F.Cu F.Paste F.Mask) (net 5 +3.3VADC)))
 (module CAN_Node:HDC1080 (layer F.Cu) (at 145 117 270)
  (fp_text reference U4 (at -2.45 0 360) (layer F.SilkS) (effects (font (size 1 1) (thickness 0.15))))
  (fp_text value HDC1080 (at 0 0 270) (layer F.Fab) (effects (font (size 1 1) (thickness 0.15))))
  (pad 1 smd rect (at -1 1.5 270) (size 0.5 1) (layers F.Cu F.Paste F.Mask) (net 31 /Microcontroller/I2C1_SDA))
  (pad 2 smd rect (at 0 1.5 270) (size 0.5 1) (layers F.Cu F.Paste F.Mask) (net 2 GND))
  (pad 3 smd rect (at 1 1.5 270) (size 0.5 1) (layers F.Cu F.Paste F.Mask) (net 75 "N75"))
  (pad 6 smd rect (at -1 -1.5 270) (size 0.5 1) (layers F.Cu F.Paste F.Mask) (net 32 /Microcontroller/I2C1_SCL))
  (pad 5 smd rect (at 0 -1.5 270) (size 0.5 1) (layers F.Cu F.Paste F.Mask) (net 11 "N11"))
  (pad 4 smd rect (at 1 -1.5 270) (size 0.5 1) (layers F.Cu F.Paste F.Mask) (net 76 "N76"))
  (pad "" smd rect (at 0 0 270) (size 2.5 1.6) (layers F.Cu F.Paste F.Mask))
  (pad "" smd rect (at 0 0 270) (size 2.5 1.6) (layers B.Cu B.Paste B.Mask))
  (pad "" thru_hole circle (at -1 -0.5 270) (size 0.5 0.5) (drill 0.2) (layers *.Cu *.Mask))
  (pad "" thru_hole circle (at 1 -0.5 270) (size 0.5 0.5) (drill 0.2) (layers *.Cu *.Mask))
  (pad "" thru_hole circle (at 0 -0.5 270) (size 0.5 0.5) (drill 0.2) (layers *.Cu *.Mask))
  (pad "" thru_hole circle (at -1 0.5 270) (size 0.5 0.5) (drill 0.2) (layers *.Cu *.Mask))
  (pad "" thru_hole circle (at 1 0.5 270) (size 0.5 0.5) (drill 0.2) (layers *.Cu *.Mask))
  (pad "" thru_hole circle (at 0 0.5 270) (size 0.5 0.5) (drill 0.2) (layers *.Cu *.Mask)))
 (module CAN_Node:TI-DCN (layer F.Cu) (at 145 85.8)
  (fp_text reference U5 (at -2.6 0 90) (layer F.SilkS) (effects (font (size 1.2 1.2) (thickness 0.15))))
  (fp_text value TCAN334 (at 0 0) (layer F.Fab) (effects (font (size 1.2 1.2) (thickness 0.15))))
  (pad 8 smd rect (at -0.975 -1.3) (size 0.45 0.9) (layers F.Cu F.Paste F.Mask) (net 70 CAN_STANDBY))
  (pad 1 smd rect (at -0.975 1.3) (size 0.45 0.9) (layers F.Cu F.Paste F.Mask) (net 74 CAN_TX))
  (pad 7 smd rect (at -0.325 -1.3) (size 0.45 0.9) (layers F.Cu F.Paste F.Mask) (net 19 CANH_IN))
  (pad 2 smd rect (at -0.325 1.3) (size 0.45 0.9) (layers F.Cu F.Paste F.Mask) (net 2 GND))
  (pad 6 smd rect (at 0.325 -1.3) (size 0.45 0.9) (layers F.Cu F.Paste F.Mask) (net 26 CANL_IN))
  (pad 3 smd rect (at 0.325 1.3) (size 0.45 0.9) (layers F.Cu F.Paste F.Mask) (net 5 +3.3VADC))
  (pad 5 smd rect (at 0.975 -1.3) (size 0.45 0.9) (layers F.Cu F.Paste F.Mask) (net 69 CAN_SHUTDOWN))
  (pad 4 smd rect (at 0.975 1.3) (size 0.45 0.9) (layers F.Cu F.Paste F.Mask) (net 73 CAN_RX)))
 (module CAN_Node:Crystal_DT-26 (layer F.Cu) (at 136.2507 113)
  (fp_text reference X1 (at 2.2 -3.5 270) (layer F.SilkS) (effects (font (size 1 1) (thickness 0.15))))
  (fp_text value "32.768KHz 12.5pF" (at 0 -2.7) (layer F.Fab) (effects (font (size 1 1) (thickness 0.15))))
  (pad 1 thru_hole circle (at -0.7493 0) (size 1.00076 1.00076) (drill 0.59944) (layers *.Cu *.Mask F.SilkS) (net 6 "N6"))
  (pad 2 thru_hole circle (at 0.7493 0) (size 1.00076 1.00076) (drill 0.59944) (layers *.Cu *.Mask F.SilkS)))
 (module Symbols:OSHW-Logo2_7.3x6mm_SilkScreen (layer F.Cu) (at 166 116.5)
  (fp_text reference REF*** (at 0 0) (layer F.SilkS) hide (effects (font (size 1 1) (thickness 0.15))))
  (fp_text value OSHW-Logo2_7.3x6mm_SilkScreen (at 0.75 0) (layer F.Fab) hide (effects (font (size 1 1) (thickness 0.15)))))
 (gr_line (start 150 120) (end 170 120) (layer Edge.Cuts) (width 0.1))
 (gr_line (start 141 120) (end 149 120) (layer Edge.Cuts) (width 0.1))
 (gr_line (start 147 112.5) (end 147 113.5) (layer Edge.Cuts) (width 0.1))
 (gr_line (start 150 112.5) (end 147 112.5) (layer Edge.Cuts) (width 0.1))
 (gr_line (start 150 120) (end 150 112.5) (layer Edge.Cuts) (width 0.1))
 (gr_line (start 140 112.5) (end 140 120) (layer Edge.Cuts) (width 0.1))
 (gr_line (start 143 112.5) (end 140 112.5) (layer Edge.Cuts) (width 0.1))
 (gr_line (start 143 113.5) (end 143 112.5) (layer Edge.Cuts) (width 0.1))
 (gr_line (start 149 113.5) (end 149 120) (layer Edge.Cuts) (width 0.1))
 (gr_line (start 147 113.5) (end 149 113.5) (layer Edge.Cuts) (width 0.1))
 (gr_line (start 141 113.5) (end 143 113.5) (layer Edge.Cuts) (width 0.1))
 (gr_line (start 141 120) (end 141 113.5) (layer Edge.Cuts) (width 0.1))
 (gr_line (start 140 120) (end 120 120) (layer Edge.Cuts) (width 0.1))
 (gr_line (start 170 80) (end 170 120) (layer Edge.Cuts) (width 0.1))
 (gr_line (start 120 80) (end 170 80) (layer Edge.Cuts) (width 0.1))
 (gr_line (start 120 120) (end 120 80) (layer Edge.Cuts) (width 0.1))
 (segment (start 142.5 117) (end 142.5 115.5) (width 0.25) (layer F.Cu) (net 2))
 (segment (start 142.5 115.5) (end 144 114) (width 0.25) (layer F.Cu) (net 2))
 (segment (start 144 114) (end 144 112) (width 0.25) (layer F.Cu) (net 2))
 (segment (start 142.5 118.335002) (end 142.5 117) (width 0.25) (layer F.Cu) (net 2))
 (segment (start 143.5 117) (end 142.5 117) (width 0.25) (layer F.Cu) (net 2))
 (segment (start 147.1 119) (end 143.164998 119) (width 0.25) (layer F.Cu) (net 2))
 (segment (start 143.164998 119) (end 142.5 118.335002) (width 0.25) (layer F.Cu) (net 2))
 (segment (start 148 118.05) (end 148 118.1) (width 0.25) (layer F.Cu) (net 2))
 (segment (start 148 118.1) (end 147.1 119) (width 0.25) (layer F.Cu) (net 2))
 (segment (start 146 113) (end 146 112) (width 0.25) (layer F.Cu) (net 11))
 (segment (start 148 115) (end 146 113) (width 0.25) (layer F.Cu) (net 11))
 (segment (start 148 116.95) (end 148 115) (width 0.25) (layer F.Cu) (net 11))
 (segment (start 146.5 117) (end 147.95 117) (width 0.25) (layer F.Cu) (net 11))
 (segment (start 147.95 117) (end 148 116.95) (width 0.25) (layer F.Cu) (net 11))
 (segment (start 144.5 114.5) (end 144.5 112) (width 0.25) (layer F.Cu) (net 31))
 (segment (start 143.5 116) (end 143.5 115.5) (width 0.25) (layer F.Cu) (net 31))
 (segment (start 143.5 115.5) (end 144.5 114.5) (width 0.25) (layer F.Cu) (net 31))
 (segment (start 145.5 114.5) (end 145.5 112) (width 0.25) (layer F.Cu) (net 32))
 (segment (start 146.5 115.5) (end 145.5 114.5) (width 0.25) (layer F.Cu) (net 32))
 (segment (start 146.5 116) (end 146.5 115.5) (width 0.25) (layer F.Cu) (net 32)))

